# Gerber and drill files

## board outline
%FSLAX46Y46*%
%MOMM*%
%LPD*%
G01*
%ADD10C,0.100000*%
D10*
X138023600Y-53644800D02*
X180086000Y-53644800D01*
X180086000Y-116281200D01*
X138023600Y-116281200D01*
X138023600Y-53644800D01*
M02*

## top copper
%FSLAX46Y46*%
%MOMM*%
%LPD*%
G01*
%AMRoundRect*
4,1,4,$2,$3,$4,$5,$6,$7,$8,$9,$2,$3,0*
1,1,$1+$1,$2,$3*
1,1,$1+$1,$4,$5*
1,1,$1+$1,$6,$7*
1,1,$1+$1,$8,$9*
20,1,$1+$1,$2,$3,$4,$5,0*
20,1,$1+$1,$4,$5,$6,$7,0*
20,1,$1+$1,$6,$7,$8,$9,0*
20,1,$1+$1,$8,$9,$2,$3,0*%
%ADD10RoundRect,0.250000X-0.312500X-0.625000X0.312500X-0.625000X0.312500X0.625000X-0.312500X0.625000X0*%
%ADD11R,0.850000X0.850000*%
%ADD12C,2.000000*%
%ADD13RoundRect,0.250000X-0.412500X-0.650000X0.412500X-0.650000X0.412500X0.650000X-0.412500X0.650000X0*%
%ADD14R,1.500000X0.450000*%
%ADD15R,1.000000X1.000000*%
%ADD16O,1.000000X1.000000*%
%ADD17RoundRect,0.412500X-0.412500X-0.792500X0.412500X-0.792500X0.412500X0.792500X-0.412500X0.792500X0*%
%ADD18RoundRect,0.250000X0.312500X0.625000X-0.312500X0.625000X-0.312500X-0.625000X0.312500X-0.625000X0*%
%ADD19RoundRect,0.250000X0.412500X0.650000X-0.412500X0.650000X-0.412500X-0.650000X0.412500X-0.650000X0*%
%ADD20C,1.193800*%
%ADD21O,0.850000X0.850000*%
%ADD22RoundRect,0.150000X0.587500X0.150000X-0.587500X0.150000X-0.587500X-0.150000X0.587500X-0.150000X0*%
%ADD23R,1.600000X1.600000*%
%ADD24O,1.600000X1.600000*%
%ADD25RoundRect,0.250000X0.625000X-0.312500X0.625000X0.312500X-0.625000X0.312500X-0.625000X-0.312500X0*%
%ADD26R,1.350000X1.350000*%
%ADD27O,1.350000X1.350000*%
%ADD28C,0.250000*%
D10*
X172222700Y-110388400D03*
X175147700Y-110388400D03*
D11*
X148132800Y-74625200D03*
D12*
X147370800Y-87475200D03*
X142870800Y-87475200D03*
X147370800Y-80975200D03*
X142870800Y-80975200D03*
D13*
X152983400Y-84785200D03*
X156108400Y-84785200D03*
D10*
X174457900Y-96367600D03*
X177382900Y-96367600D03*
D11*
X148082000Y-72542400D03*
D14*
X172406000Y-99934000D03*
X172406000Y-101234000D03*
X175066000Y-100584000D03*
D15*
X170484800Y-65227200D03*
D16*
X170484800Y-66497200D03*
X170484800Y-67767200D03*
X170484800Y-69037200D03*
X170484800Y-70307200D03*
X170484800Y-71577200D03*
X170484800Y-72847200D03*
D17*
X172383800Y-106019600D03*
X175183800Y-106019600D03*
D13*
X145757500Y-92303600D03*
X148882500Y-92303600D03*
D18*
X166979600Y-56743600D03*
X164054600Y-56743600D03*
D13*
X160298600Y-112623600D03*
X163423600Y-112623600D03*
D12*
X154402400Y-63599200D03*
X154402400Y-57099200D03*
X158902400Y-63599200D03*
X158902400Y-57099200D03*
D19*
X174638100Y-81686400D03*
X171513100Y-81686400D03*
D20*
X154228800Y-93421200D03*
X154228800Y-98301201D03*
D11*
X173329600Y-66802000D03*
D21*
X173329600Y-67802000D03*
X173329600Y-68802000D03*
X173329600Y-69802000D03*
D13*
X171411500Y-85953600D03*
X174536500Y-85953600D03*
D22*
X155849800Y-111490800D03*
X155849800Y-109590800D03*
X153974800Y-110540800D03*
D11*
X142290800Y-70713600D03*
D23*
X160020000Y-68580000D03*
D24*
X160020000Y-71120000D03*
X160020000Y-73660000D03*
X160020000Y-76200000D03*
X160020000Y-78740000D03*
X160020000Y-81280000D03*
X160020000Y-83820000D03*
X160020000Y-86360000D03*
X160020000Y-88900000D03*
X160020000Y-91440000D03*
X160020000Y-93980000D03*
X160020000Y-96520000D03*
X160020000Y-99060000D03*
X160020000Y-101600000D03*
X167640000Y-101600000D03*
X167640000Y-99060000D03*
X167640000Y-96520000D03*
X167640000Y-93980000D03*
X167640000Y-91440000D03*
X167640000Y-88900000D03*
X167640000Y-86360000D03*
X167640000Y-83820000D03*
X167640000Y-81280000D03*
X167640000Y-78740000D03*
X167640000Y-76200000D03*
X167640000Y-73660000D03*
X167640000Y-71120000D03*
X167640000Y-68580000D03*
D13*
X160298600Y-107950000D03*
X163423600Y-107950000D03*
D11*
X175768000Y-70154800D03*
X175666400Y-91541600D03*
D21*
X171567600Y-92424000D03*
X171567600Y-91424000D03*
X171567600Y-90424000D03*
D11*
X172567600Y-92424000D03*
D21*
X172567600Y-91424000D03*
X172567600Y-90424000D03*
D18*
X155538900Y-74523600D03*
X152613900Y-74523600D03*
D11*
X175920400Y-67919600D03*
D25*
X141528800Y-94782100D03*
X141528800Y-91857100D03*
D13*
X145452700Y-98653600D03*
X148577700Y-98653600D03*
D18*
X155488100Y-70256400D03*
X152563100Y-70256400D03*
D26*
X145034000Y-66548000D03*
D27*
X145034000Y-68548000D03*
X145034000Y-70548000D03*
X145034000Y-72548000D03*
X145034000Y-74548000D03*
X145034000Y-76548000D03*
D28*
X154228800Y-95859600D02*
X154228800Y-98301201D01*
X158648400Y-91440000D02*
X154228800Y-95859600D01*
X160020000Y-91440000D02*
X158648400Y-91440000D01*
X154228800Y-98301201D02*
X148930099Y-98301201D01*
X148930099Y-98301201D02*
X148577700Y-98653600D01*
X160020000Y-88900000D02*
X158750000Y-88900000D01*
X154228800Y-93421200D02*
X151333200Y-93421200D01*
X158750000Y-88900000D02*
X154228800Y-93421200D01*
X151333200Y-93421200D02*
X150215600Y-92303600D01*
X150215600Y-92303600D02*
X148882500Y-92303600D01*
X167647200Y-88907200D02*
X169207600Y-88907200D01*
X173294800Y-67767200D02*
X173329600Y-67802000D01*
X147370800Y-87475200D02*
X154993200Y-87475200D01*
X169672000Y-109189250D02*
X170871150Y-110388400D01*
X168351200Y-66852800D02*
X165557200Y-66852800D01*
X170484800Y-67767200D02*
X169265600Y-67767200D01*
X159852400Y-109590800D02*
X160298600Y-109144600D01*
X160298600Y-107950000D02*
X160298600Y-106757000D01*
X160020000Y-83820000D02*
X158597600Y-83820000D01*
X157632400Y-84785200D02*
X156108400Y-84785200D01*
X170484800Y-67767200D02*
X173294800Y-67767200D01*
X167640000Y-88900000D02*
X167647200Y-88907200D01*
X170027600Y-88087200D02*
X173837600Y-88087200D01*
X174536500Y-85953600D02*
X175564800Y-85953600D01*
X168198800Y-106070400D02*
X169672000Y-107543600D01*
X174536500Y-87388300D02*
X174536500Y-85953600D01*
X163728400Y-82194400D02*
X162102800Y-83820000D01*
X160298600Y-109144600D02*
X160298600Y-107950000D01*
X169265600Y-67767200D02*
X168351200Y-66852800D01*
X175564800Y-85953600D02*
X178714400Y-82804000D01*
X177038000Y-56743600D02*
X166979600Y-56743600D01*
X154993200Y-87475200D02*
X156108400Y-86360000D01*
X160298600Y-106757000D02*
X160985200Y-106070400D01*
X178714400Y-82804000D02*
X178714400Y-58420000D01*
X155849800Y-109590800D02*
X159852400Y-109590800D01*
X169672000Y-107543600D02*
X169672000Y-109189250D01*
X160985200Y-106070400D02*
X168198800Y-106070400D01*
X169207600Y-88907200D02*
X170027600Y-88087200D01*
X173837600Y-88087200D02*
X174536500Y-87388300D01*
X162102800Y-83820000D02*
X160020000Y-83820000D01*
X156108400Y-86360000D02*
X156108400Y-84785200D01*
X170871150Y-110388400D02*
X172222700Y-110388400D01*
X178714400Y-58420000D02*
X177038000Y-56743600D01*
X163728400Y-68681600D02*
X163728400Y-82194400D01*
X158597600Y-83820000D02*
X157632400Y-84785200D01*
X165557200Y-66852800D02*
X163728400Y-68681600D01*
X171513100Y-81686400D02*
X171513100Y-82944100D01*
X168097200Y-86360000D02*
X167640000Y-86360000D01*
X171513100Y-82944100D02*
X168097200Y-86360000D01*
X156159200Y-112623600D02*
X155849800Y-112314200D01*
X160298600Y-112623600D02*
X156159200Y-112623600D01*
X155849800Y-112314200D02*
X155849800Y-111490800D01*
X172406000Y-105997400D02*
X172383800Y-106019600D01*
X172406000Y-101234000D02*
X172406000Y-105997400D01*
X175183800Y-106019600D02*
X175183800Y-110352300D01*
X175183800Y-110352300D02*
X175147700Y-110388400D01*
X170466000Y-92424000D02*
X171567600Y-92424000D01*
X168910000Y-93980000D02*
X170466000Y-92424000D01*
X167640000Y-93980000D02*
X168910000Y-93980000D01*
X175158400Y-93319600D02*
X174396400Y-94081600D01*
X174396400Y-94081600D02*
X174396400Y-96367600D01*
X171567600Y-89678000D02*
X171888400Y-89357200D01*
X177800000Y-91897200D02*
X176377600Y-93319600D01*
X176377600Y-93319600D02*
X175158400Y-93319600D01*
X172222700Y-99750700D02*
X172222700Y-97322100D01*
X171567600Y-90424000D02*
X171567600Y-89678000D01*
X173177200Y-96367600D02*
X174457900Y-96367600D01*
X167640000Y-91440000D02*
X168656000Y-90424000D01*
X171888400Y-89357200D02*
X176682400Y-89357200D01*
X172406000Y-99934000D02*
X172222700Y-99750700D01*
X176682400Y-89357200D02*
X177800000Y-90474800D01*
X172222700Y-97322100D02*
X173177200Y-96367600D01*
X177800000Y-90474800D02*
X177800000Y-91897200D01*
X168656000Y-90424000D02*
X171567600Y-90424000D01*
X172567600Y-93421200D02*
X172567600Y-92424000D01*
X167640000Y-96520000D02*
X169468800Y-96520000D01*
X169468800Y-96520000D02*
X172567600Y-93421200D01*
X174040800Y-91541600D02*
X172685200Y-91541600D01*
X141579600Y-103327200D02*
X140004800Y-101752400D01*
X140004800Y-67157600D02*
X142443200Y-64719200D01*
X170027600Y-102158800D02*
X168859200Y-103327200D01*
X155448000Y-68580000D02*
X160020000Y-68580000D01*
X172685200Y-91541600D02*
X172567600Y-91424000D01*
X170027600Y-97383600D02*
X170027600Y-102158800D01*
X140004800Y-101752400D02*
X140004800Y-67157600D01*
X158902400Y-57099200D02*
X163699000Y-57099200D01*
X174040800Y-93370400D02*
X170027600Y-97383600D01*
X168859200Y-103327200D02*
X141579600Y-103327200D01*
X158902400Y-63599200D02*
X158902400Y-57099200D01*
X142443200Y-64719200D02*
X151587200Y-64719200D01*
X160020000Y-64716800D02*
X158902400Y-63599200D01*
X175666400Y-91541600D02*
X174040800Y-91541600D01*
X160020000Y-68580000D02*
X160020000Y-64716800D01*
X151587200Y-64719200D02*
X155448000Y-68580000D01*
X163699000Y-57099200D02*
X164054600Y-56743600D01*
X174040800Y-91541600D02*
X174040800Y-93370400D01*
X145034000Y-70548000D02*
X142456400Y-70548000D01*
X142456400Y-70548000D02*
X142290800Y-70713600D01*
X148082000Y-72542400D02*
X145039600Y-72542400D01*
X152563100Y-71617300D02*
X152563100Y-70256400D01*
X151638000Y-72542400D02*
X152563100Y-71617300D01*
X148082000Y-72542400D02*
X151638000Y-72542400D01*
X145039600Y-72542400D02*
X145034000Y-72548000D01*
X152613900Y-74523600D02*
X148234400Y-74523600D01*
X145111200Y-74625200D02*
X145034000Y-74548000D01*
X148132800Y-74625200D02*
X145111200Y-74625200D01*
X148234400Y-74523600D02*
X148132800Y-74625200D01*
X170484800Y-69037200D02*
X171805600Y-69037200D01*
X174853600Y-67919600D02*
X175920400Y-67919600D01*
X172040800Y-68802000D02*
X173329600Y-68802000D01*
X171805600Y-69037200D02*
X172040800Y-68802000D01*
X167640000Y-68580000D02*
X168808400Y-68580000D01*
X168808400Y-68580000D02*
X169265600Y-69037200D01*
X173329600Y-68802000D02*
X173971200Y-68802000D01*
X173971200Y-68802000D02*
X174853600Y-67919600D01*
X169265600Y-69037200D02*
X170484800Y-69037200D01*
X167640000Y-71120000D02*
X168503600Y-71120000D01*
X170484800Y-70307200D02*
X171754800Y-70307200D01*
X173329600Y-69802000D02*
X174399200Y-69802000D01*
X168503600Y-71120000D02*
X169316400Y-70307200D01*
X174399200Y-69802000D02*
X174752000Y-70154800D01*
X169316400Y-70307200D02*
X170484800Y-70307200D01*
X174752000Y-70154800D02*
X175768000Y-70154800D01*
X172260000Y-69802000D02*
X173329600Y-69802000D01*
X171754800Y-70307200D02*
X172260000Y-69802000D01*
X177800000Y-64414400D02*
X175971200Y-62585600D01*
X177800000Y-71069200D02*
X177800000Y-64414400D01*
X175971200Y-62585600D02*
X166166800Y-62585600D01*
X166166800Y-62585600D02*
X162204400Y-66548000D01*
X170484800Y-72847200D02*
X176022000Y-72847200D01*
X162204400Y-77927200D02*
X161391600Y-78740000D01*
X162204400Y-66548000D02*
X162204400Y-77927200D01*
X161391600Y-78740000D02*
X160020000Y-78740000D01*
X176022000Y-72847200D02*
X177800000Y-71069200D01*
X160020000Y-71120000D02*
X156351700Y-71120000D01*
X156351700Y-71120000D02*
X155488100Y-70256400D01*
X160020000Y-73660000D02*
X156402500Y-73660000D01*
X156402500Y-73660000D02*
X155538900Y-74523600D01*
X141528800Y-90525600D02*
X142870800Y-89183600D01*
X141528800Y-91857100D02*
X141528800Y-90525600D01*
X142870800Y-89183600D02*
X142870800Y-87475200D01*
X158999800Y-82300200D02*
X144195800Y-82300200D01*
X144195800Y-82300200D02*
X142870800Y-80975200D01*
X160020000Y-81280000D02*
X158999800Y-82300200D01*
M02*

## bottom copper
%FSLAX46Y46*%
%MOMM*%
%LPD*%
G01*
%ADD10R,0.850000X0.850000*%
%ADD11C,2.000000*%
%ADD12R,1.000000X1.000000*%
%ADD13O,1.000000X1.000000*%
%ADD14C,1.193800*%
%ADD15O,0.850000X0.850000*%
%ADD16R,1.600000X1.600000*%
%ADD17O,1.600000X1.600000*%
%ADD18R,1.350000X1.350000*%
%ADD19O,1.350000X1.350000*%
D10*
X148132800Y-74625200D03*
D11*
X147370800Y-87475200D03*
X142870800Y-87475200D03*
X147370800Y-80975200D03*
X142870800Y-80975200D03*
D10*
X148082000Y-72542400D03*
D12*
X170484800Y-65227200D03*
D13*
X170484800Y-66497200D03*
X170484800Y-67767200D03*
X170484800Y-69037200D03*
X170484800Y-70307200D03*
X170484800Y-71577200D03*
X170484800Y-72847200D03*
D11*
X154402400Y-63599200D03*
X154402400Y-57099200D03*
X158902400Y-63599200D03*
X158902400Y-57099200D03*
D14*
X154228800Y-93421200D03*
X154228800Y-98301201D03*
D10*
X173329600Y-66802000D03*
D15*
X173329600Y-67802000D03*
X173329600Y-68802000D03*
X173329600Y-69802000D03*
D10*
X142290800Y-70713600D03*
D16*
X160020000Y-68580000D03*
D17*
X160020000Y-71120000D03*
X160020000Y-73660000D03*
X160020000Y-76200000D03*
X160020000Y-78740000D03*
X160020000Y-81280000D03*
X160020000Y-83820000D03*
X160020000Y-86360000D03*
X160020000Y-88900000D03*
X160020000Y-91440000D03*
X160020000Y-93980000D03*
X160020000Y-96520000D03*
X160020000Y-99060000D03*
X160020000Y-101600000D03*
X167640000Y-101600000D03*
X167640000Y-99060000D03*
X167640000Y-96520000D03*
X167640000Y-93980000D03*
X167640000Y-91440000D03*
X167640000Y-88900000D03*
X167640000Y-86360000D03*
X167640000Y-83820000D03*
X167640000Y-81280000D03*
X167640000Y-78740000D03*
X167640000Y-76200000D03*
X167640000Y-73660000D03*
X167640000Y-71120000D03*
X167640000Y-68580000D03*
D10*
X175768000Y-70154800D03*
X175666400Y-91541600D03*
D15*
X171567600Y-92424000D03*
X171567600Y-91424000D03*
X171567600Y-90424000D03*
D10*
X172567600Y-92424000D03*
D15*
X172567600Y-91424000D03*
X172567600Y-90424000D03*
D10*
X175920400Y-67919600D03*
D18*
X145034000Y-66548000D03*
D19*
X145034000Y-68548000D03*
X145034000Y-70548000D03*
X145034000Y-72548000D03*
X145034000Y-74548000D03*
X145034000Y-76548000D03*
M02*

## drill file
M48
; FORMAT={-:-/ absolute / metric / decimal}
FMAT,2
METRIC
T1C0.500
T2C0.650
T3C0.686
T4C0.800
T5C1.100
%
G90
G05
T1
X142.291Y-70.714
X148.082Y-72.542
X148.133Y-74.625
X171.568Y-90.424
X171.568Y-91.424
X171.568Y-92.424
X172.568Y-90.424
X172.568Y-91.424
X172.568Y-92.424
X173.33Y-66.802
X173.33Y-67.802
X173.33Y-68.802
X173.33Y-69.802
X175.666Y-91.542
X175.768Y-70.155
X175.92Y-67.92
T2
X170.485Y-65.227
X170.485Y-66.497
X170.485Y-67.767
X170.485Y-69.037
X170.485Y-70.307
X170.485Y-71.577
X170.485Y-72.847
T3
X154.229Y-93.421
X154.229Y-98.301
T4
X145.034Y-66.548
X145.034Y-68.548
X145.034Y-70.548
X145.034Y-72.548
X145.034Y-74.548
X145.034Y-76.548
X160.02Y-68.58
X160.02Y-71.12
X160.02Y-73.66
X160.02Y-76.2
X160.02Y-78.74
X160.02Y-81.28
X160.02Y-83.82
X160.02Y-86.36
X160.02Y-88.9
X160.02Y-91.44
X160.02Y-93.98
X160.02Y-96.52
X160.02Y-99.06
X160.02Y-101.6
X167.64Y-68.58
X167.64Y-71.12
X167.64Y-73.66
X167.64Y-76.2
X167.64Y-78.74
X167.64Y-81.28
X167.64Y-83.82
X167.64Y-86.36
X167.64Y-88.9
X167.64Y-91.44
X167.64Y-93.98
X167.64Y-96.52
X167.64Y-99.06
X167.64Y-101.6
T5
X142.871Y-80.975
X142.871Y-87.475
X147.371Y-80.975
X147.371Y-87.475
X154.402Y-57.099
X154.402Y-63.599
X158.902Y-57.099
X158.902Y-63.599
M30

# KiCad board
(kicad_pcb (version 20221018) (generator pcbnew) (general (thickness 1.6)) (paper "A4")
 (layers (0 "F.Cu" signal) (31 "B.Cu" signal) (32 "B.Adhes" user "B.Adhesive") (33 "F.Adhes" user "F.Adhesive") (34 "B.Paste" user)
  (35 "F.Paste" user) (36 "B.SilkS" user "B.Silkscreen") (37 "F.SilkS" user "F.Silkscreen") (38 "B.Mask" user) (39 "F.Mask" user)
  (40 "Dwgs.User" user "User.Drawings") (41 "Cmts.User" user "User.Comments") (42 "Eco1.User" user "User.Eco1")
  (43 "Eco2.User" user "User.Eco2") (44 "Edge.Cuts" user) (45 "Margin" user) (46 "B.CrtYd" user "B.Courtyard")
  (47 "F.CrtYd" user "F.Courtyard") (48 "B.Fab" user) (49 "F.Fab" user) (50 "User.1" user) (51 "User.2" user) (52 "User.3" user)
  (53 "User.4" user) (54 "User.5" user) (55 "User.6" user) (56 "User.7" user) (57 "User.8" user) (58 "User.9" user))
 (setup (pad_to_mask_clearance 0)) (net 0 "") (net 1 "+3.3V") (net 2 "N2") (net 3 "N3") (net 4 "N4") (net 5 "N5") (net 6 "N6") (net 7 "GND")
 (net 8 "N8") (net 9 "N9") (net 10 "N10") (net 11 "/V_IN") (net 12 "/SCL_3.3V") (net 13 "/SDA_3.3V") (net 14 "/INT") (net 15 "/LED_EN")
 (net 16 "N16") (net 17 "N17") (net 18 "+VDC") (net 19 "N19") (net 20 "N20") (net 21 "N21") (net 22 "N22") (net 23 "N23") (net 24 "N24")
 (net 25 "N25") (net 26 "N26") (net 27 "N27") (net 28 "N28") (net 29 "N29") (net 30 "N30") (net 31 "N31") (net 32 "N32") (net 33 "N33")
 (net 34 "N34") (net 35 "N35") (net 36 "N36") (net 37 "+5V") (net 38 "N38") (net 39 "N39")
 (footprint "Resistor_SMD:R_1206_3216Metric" (layer "F.Cu") (at 173.6852 110.3884)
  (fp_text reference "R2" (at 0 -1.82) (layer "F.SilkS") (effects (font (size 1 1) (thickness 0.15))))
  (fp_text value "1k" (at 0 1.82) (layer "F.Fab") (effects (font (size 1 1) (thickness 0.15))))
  (pad "1" smd roundrect (at -1.4625 0) (size 1.125 1.75) (layers "F.Cu" "F.Paste" "F.Mask") (roundrect_rratio 0.222222) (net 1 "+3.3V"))
  (pad "2" smd roundrect (at 1.4625 0) (size 1.125 1.75) (layers "F.Cu" "F.Paste" "F.Mask") (roundrect_rratio 0.222222) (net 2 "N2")))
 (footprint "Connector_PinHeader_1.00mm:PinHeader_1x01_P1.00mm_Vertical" (layer "F.Cu") (at 148.1328 74.6252)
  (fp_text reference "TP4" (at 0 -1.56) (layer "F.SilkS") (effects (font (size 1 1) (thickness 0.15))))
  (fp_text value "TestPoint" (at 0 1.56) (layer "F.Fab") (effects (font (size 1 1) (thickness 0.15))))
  (pad "1" thru_hole rect (at 0 0) (size 0.85 0.85) (drill 0.5) (layers "*.Cu" "*.Mask") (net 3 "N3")))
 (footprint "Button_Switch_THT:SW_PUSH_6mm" (layer "F.Cu") (at 147.3708 80.9752 -90)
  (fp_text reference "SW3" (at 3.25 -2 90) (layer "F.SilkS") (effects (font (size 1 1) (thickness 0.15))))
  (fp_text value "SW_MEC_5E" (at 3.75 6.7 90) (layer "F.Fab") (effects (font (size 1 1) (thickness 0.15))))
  (pad "1" thru_hole circle (at 6.5 0) (size 2 2) (drill 1.1) (layers "*.Cu" "*.Mask") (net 1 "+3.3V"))
  (pad "2" thru_hole circle (at 6.5 4.5) (size 2 2) (drill 1.1) (layers "*.Cu" "*.Mask") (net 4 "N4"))
  (pad "3" thru_hole circle (at 0 0) (size 2 2) (drill 1.1) (layers "*.Cu" "*.Mask") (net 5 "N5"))
  (pad "4" thru_hole circle (at 0 4.5) (size 2 2) (drill 1.1) (layers "*.Cu" "*.Mask") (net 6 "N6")))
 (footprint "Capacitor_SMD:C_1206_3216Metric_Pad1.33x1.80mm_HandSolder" (layer "F.Cu") (at 154.5459 84.7852)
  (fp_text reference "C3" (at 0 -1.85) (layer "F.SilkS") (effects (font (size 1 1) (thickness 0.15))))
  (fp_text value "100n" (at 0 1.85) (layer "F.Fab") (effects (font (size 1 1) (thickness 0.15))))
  (pad "1" smd roundrect (at -1.5625 0) (size 1.325 1.8) (layers "F.Cu" "F.Paste" "F.Mask") (roundrect_rratio 0.188679) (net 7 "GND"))
  (pad "2" smd roundrect (at 1.5625 0) (size 1.325 1.8) (layers "F.Cu" "F.Paste" "F.Mask") (roundrect_rratio 0.188679) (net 1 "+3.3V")))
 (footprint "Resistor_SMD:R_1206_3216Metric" (layer "F.Cu") (at 175.9204 96.3676)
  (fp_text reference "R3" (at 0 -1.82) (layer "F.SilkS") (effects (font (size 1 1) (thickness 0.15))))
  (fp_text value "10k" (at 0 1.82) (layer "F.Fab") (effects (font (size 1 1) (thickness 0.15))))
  (pad "1" smd roundrect (at -1.4625 0) (size 1.125 1.75) (layers "F.Cu" "F.Paste" "F.Mask") (roundrect_rratio 0.222222) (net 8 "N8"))
  (pad "2" smd roundrect (at 1.4625 0) (size 1.125 1.75) (layers "F.Cu" "F.Paste" "F.Mask") (roundrect_rratio 0.222222) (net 7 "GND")))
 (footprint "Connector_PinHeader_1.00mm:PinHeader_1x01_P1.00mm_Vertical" (layer "F.Cu") (at 148.082 72.5424)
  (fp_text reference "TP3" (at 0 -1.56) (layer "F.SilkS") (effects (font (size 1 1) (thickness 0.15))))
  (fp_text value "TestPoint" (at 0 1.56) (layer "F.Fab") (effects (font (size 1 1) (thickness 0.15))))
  (pad "1" thru_hole rect (at 0 0) (size 0.85 0.85) (drill 0.5) (layers "*.Cu" "*.Mask") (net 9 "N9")))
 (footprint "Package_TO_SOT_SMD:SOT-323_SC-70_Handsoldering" (layer "F.Cu") (at 173.736 100.584)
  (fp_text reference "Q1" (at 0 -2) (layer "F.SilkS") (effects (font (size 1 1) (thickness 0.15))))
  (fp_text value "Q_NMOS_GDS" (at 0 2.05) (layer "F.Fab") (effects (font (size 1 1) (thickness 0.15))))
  (pad "1" smd rect (at -1.33 -0.65 270) (size 0.45 1.5) (layers "F.Cu" "F.Paste" "F.Mask") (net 8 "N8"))
  (pad "2" smd rect (at -1.33 0.65 270) (size 0.45 1.5) (layers "F.Cu" "F.Paste" "F.Mask") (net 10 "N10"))
  (pad "3" smd rect (at 1.33 0 270) (size 0.45 1.5) (layers "F.Cu" "F.Paste" "F.Mask") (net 7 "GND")))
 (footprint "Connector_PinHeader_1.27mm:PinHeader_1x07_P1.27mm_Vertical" (layer "F.Cu") (at 170.4848 65.2272)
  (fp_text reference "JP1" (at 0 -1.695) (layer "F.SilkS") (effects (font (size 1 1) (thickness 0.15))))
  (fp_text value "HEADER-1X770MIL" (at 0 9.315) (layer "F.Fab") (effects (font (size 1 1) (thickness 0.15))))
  (pad "1" thru_hole rect (at 0 0) (size 1 1) (drill 0.65) (layers "*.Cu" "*.Mask") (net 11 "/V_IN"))
  (pad "2" thru_hole oval (at 0 1.27) (size 1 1) (drill 0.65) (layers "*.Cu" "*.Mask") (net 7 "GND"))
  (pad "3" thru_hole oval (at 0 2.54) (size 1 1) (drill 0.65) (layers "*.Cu" "*.Mask") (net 1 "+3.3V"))
  (pad "4" thru_hole oval (at 0 3.81) (size 1 1) (drill 0.65) (layers "*.Cu" "*.Mask") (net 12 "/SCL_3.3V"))
  (pad "5" thru_hole oval (at 0 5.08) (size 1 1) (drill 0.65) (layers "*.Cu" "*.Mask") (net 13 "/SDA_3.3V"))
  (pad "6" thru_hole oval (at 0 6.35) (size 1 1) (drill 0.65) (layers "*.Cu" "*.Mask") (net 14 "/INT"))
  (pad "7" thru_hole oval (at 0 7.62) (size 1 1) (drill 0.65) (layers "*.Cu" "*.Mask") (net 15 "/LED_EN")))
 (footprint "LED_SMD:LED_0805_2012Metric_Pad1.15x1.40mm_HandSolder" (layer "F.Cu") (at 173.7868 106.0196)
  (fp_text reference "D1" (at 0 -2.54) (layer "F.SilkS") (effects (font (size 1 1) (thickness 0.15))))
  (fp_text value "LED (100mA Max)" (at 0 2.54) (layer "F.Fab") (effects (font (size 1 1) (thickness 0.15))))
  (pad "1" smd roundrect (at -1.403 0) (size 1.65 2.41) (layers "F.Cu" "F.Paste" "F.Mask") (roundrect_rratio 0.25) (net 10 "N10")
   (thermal_bridge_angle 45))
  (pad "2" smd roundrect (at 1.397 0) (size 1.65 2.41) (layers "F.Cu" "F.Paste" "F.Mask") (roundrect_rratio 0.25) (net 2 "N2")
   (thermal_bridge_angle 45)))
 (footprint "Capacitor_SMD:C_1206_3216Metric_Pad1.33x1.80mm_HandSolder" (layer "F.Cu") (at 147.32 92.3036)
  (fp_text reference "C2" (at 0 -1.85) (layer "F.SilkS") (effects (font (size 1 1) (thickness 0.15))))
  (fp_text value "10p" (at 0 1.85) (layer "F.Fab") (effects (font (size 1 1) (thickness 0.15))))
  (pad "1" smd roundrect (at -1.5625 0) (size 1.325 1.8) (layers "F.Cu" "F.Paste" "F.Mask") (roundrect_rratio 0.188679) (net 7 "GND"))
  (pad "2" smd roundrect (at 1.5625 0) (size 1.325 1.8) (layers "F.Cu" "F.Paste" "F.Mask") (roundrect_rratio 0.188679) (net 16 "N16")))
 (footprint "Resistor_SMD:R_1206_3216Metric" (layer "F.Cu") (at 165.5171 56.7436 180)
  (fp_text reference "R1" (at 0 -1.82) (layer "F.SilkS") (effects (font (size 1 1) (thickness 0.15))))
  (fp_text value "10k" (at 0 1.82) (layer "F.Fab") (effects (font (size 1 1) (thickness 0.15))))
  (pad "1" smd roundrect (at -1.4625 0 180) (size 1.125 1.75) (layers "F.Cu" "F.Paste" "F.Mask") (roundrect_rratio 0.222222) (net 1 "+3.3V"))
  (pad "2" smd roundrect (at 1.4625 0 180) (size 1.125 1.75) (layers "F.Cu" "F.Paste" "F.Mask") (roundrect_rratio 0.222222) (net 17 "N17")))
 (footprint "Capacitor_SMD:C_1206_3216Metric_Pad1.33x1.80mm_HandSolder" (layer "F.Cu") (at 161.8611 112.6236)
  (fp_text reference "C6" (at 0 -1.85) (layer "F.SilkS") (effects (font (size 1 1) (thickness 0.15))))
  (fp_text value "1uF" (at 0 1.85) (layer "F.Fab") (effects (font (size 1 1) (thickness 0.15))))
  (pad "1" smd roundrect (at -1.5625 0) (size 1.325 1.8) (layers "F.Cu" "F.Paste" "F.Mask") (roundrect_rratio 0.188679) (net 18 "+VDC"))
  (pad "2" smd roundrect (at 1.5625 0) (size 1.325 1.8) (layers "F.Cu" "F.Paste" "F.Mask") (roundrect_rratio 0.188679) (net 7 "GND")))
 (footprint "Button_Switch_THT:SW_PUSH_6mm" (layer "F.Cu") (at 154.4024 63.5992 90)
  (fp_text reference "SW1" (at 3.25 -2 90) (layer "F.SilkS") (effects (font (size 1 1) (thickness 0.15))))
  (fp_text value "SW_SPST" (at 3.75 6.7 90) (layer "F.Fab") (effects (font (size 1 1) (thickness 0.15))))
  (pad "1" thru_hole circle (at 0 0 180) (size 2 2) (drill 1.1) (layers "*.Cu" "*.Mask") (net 7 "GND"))
  (pad "1" thru_hole circle (at 6.5 0 180) (size 2 2) (drill 1.1) (layers "*.Cu" "*.Mask") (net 7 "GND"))
  (pad "2" thru_hole circle (at 0 4.5 180) (size 2 2) (drill 1.1) (layers "*.Cu" "*.Mask") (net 17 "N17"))
  (pad "2" thru_hole circle (at 6.5 4.5 180) (size 2 2) (drill 1.1) (layers "*.Cu" "*.Mask") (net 17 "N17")))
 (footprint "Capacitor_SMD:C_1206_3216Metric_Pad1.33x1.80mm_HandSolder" (layer "F.Cu") (at 173.0756 81.6864 180)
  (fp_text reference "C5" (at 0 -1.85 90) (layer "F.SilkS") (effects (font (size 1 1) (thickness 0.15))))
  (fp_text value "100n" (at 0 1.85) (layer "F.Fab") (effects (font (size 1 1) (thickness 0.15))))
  (pad "1" smd roundrect (at -1.5625 0 180) (size 1.325 1.8) (layers "F.Cu" "F.Paste" "F.Mask") (roundrect_rratio 0.188679) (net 7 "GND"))
  (pad "2" smd roundrect (at 1.5625 0 180) (size 1.325 1.8) (layers "F.Cu" "F.Paste" "F.Mask") (roundrect_rratio 0.188679) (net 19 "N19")))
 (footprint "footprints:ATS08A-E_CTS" (layer "F.Cu") (at 154.2288 93.4212 -90)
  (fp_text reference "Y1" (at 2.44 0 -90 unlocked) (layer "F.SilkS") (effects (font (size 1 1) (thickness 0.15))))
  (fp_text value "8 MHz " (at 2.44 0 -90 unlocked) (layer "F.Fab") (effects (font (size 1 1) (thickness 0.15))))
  (pad "1" thru_hole circle (at 0 0 270) (size 1.1938 1.1938) (drill 0.6858) (layers "*.Cu" "*.Mask") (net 16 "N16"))
  (pad "2" thru_hole circle (at 4.880001 0 270) (size 1.1938 1.1938) (drill 0.6858) (layers "*.Cu" "*.Mask") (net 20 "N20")))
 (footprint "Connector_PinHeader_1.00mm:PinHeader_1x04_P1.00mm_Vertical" (layer "F.Cu") (at 173.3296 66.802)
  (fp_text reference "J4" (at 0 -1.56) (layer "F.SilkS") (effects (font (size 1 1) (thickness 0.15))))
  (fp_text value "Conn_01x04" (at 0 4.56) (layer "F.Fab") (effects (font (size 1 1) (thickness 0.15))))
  (pad "1" thru_hole rect (at 0 0) (size 0.85 0.85) (drill 0.5) (layers "*.Cu" "*.Mask") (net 7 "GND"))
  (pad "2" thru_hole oval (at 0 1) (size 0.85 0.85) (drill 0.5) (layers "*.Cu" "*.Mask") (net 1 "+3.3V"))
  (pad "3" thru_hole oval (at 0 2) (size 0.85 0.85) (drill 0.5) (layers "*.Cu" "*.Mask") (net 12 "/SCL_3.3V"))
  (pad "4" thru_hole oval (at 0 3) (size 0.85 0.85) (drill 0.5) (layers "*.Cu" "*.Mask") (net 13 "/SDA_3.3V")))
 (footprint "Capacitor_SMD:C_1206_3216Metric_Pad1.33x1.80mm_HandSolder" (layer "F.Cu") (at 172.974 85.9536)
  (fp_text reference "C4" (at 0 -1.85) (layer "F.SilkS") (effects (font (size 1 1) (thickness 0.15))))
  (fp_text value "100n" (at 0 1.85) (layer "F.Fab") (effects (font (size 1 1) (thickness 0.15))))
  (pad "1" smd roundrect (at -1.5625 0) (size 1.325 1.8) (layers "F.Cu" "F.Paste" "F.Mask") (roundrect_rratio 0.188679) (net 7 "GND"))
  (pad "2" smd roundrect (at 1.5625 0) (size 1.325 1.8) (layers "F.Cu" "F.Paste" "F.Mask") (roundrect_rratio 0.188679) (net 1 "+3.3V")))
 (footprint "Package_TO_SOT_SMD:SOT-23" (layer "F.Cu") (at 154.9123 110.5408 180)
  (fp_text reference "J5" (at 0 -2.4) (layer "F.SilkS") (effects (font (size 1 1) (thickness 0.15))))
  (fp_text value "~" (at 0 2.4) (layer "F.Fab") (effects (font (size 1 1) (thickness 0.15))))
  (pad "1" smd roundrect (at -0.9375 -0.95 180) (size 1.475 0.6) (layers "F.Cu" "F.Paste" "F.Mask") (roundrect_rratio 0.25) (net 18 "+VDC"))
  (pad "2" smd roundrect (at -0.9375 0.95 180) (size 1.475 0.6) (layers "F.Cu" "F.Paste" "F.Mask") (roundrect_rratio 0.25) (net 1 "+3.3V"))
  (pad "3" smd roundrect (at 0.9375 0 180) (size 1.475 0.6) (layers "F.Cu" "F.Paste" "F.Mask") (roundrect_rratio 0.25) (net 7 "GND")))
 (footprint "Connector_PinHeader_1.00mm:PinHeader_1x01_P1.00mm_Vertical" (layer "F.Cu") (at 142.2908 70.7136)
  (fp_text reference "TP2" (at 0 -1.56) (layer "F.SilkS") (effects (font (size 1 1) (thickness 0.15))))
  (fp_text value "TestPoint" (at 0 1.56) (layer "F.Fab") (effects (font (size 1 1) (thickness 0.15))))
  (pad "1" thru_hole rect (at 0 0) (size 0.85 0.85) (drill 0.5) (layers "*.Cu" "*.Mask") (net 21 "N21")))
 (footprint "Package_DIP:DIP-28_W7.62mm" (layer "F.Cu") (at 160.02 68.58)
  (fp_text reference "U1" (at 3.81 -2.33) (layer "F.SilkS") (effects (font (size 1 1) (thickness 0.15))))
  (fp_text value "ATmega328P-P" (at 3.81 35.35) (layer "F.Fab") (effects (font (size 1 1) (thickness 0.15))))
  (pad "1" thru_hole rect (at 0 0) (size 1.6 1.6) (drill 0.8) (layers "*.Cu" "*.Mask") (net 17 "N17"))
  (pad "2" thru_hole oval (at 0 2.54) (size 1.6 1.6) (drill 0.8) (layers "*.Cu" "*.Mask") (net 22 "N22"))
  (pad "3" thru_hole oval (at 0 5.08) (size 1.6 1.6) (drill 0.8) (layers "*.Cu" "*.Mask") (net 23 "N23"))
  (pad "4" thru_hole oval (at 0 7.62) (size 1.6 1.6) (drill 0.8) (layers "*.Cu" "*.Mask") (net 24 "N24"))
  (pad "5" thru_hole oval (at 0 10.16) (size 1.6 1.6) (drill 0.8) (layers "*.Cu" "*.Mask") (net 15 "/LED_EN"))
  (pad "6" thru_hole oval (at 0 12.7) (size 1.6 1.6) (drill 0.8) (layers "*.Cu" "*.Mask") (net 6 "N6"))
  (pad "7" thru_hole oval (at 0 15.24) (size 1.6 1.6) (drill 0.8) (layers "*.Cu" "*.Mask") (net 1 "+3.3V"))
  (pad "8" thru_hole oval (at 0 17.78) (size 1.6 1.6) (drill 0.8) (layers "*.Cu" "*.Mask") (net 7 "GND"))
  (pad "9" thru_hole oval (at 0 20.32) (size 1.6 1.6) (drill 0.8) (layers "*.Cu" "*.Mask") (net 16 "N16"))
  (pad "10" thru_hole oval (at 0 22.86) (size 1.6 1.6) (drill 0.8) (layers "*.Cu" "*.Mask") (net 20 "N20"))
  (pad "11" thru_hole oval (at 0 25.4) (size 1.6 1.6) (drill 0.8) (layers "*.Cu" "*.Mask") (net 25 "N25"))
  (pad "12" thru_hole oval (at 0 27.94) (size 1.6 1.6) (drill 0.8) (layers "*.Cu" "*.Mask") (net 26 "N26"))
  (pad "13" thru_hole oval (at 0 30.48) (size 1.6 1.6) (drill 0.8) (layers "*.Cu" "*.Mask") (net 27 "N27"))
  (pad "14" thru_hole oval (at 0 33.02) (size 1.6 1.6) (drill 0.8) (layers "*.Cu" "*.Mask") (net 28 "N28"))
  (pad "15" thru_hole oval (at 7.62 33.02) (size 1.6 1.6) (drill 0.8) (layers "*.Cu" "*.Mask") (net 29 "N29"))
  (pad "16" thru_hole oval (at 7.62 30.48) (size 1.6 1.6) (drill 0.8) (layers "*.Cu" "*.Mask") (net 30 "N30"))
  (pad "17" thru_hole oval (at 7.62 27.94) (size 1.6 1.6) (drill 0.8) (layers "*.Cu" "*.Mask") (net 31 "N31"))
  (pad "18" thru_hole oval (at 7.62 25.4) (size 1.6 1.6) (drill 0.8) (layers "*.Cu" "*.Mask") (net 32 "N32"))
  (pad "19" thru_hole oval (at 7.62 22.86) (size 1.6 1.6) (drill 0.8) (layers "*.Cu" "*.Mask") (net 8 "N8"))
  (pad "20" thru_hole oval (at 7.62 20.32) (size 1.6 1.6) (drill 0.8) (layers "*.Cu" "*.Mask") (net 1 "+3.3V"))
  (pad "21" thru_hole oval (at 7.62 17.78) (size 1.6 1.6) (drill 0.8) (layers "*.Cu" "*.Mask") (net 19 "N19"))
  (pad "22" thru_hole oval (at 7.62 15.24) (size 1.6 1.6) (drill 0.8) (layers "*.Cu" "*.Mask") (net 7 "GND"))
  (pad "23" thru_hole oval (at 7.62 12.7) (size 1.6 1.6) (drill 0.8) (layers "*.Cu" "*.Mask") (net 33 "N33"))
  (pad "24" thru_hole oval (at 7.62 10.16) (size 1.6 1.6) (drill 0.8) (layers "*.Cu" "*.Mask") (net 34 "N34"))
  (pad "25" thru_hole oval (at 7.62 7.62) (size 1.6 1.6) (drill 0.8) (layers "*.Cu" "*.Mask") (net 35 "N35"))
  (pad "26" thru_hole oval (at 7.62 5.08) (size 1.6 1.6) (drill 0.8) (layers "*.Cu" "*.Mask") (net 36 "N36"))
  (pad "27" thru_hole oval (at 7.62 2.54) (size 1.6 1.6) (drill 0.8) (layers "*.Cu" "*.Mask") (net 13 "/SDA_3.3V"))
  (pad "28" thru_hole oval (at 7.62 0) (size 1.6 1.6) (drill 0.8) (layers "*.Cu" "*.Mask") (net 12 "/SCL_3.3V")))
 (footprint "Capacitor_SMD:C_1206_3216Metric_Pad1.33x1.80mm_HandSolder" (layer "F.Cu") (at 161.8611 107.95)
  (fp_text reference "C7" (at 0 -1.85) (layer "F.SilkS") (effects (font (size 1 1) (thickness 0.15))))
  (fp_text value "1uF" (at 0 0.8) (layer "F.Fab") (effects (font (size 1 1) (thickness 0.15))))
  (pad "1" smd roundrect (at -1.5625 0) (size 1.325 1.8) (layers "F.Cu" "F.Paste" "F.Mask") (roundrect_rratio 0.188679) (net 1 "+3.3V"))
  (pad "2" smd roundrect (at 1.5625 0) (size 1.325 1.8) (layers "F.Cu" "F.Paste" "F.Mask") (roundrect_rratio 0.188679) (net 7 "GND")))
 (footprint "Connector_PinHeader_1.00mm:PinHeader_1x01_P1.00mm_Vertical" (layer "F.Cu") (at 175.768 70.1548)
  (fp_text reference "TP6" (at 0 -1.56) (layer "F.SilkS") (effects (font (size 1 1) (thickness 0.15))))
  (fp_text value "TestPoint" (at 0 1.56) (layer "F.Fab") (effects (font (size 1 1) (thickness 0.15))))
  (pad "1" thru_hole rect (at 0 0) (size 0.85 0.85) (drill 0.5) (layers "*.Cu" "*.Mask") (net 13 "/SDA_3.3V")))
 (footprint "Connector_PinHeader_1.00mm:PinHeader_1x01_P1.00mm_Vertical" (layer "F.Cu") (at 175.6664 91.5416)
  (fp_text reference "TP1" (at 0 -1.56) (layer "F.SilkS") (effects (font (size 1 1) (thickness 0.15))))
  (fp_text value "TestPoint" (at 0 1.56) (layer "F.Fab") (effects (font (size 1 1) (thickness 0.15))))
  (pad "1" thru_hole rect (at 0 0) (size 0.85 0.85) (drill 0.5) (layers "*.Cu" "*.Mask") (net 17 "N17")))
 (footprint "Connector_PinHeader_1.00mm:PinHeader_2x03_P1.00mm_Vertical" (layer "F.Cu") (at 172.5676 92.424 180)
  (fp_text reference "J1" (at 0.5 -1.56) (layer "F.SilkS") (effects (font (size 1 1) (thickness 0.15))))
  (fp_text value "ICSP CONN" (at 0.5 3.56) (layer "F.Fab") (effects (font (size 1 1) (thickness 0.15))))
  (pad "1" thru_hole oval (at 1 0 180) (size 0.85 0.85) (drill 0.5) (layers "*.Cu" "*.Mask") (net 32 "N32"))
  (pad "2" thru_hole oval (at 1 1 180) (size 0.85 0.85) (drill 0.5) (layers "*.Cu" "*.Mask") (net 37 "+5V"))
  (pad "3" thru_hole oval (at 1 2 180) (size 0.85 0.85) (drill 0.5) (layers "*.Cu" "*.Mask") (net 8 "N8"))
  (pad "4" thru_hole rect (at 0 0 180) (size 0.85 0.85) (drill 0.5) (layers "*.Cu" "*.Mask") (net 31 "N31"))
  (pad "5" thru_hole oval (at 0 1 180) (size 0.85 0.85) (drill 0.5) (layers "*.Cu" "*.Mask") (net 17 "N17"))
  (pad "6" thru_hole oval (at 0 2 180) (size 0.85 0.85) (drill 0.5) (layers "*.Cu" "*.Mask") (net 7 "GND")))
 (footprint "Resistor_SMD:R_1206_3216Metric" (layer "F.Cu") (at 154.0764 74.5236 180)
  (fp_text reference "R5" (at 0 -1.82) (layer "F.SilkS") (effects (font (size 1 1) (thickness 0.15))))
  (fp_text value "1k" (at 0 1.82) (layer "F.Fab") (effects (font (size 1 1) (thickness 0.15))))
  (pad "1" smd roundrect (at -1.4625 0 180) (size 1.125 1.75) (layers "F.Cu" "F.Paste" "F.Mask") (roundrect_rratio 0.222222) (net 23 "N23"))
  (pad "2" smd roundrect (at 1.4625 0 180) (size 1.125 1.75) (layers "F.Cu" "F.Paste" "F.Mask") (roundrect_rratio 0.222222) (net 3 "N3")))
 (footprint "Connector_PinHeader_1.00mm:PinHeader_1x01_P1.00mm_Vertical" (layer "F.Cu") (at 175.9204 67.9196)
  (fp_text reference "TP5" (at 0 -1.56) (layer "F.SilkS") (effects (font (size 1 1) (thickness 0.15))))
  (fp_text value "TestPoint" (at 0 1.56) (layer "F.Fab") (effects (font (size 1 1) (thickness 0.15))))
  (pad "1" thru_hole rect (at 0 0) (size 0.85 0.85) (drill 0.5) (layers "*.Cu" "*.Mask") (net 12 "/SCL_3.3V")))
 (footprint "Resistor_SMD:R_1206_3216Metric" (layer "F.Cu") (at 141.5288 93.3196 90)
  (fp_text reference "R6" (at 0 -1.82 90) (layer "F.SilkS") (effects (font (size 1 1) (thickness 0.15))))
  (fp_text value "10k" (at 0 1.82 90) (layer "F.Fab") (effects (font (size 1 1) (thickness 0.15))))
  (pad "1" smd roundrect (at -1.4625 0 90) (size 1.125 1.75) (layers "F.Cu" "F.Paste" "F.Mask") (roundrect_rratio 0.222222) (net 7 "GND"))
  (pad "2" smd roundrect (at 1.4625 0 90) (size 1.125 1.75) (layers "F.Cu" "F.Paste" "F.Mask") (roundrect_rratio 0.222222) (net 4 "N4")))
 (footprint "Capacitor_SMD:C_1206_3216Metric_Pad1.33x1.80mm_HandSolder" (layer "F.Cu") (at 147.0152 98.6536)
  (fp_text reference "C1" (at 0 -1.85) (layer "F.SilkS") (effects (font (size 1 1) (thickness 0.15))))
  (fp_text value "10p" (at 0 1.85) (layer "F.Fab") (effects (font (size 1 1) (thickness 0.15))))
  (pad "1" smd roundrect (at -1.5625 0) (size 1.325 1.8) (layers "F.Cu" "F.Paste" "F.Mask") (roundrect_rratio 0.188679) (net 7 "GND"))
  (pad "2" smd roundrect (at 1.5625 0) (size 1.325 1.8) (layers "F.Cu" "F.Paste" "F.Mask") (roundrect_rratio 0.188679) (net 20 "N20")))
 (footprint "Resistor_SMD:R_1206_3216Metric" (layer "F.Cu") (at 154.0256 70.2564 180)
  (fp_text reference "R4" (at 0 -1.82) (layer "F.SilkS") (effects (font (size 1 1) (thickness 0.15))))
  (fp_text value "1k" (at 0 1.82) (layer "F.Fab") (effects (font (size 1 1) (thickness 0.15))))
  (pad "1" smd roundrect (at -1.4625 0 180) (size 1.125 1.75) (layers "F.Cu" "F.Paste" "F.Mask") (roundrect_rratio 0.222222) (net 22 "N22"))
  (pad "2" smd roundrect (at 1.4625 0 180) (size 1.125 1.75) (layers "F.Cu" "F.Paste" "F.Mask") (roundrect_rratio 0.222222) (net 9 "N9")))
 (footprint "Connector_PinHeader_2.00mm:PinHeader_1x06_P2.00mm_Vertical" (layer "F.Cu") (at 145.034 66.548)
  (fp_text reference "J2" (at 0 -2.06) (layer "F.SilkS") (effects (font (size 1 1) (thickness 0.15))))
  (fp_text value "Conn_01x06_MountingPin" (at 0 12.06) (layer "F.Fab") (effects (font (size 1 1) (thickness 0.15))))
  (pad "1" thru_hole rect (at 0 0) (size 1.35 1.35) (drill 0.8) (layers "*.Cu" "*.Mask") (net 7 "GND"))
  (pad "2" thru_hole oval (at 0 2) (size 1.35 1.35) (drill 0.8) (layers "*.Cu" "*.Mask") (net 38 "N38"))
  (pad "3" thru_hole oval (at 0 4) (size 1.35 1.35) (drill 0.8) (layers "*.Cu" "*.Mask") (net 21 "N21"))
  (pad "4" thru_hole oval (at 0 6) (size 1.35 1.35) (drill 0.8) (layers "*.Cu" "*.Mask") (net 9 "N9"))
  (pad "5" thru_hole oval (at 0 8) (size 1.35 1.35) (drill 0.8) (layers "*.Cu" "*.Mask") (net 3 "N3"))
  (pad "6" thru_hole oval (at 0 10) (size 1.35 1.35) (drill 0.8) (layers "*.Cu" "*.Mask") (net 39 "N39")))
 (gr_rect (start 138.0236 53.6448) (end 180.086 116.2812) (stroke (width 0.1) (type default)) (fill none) (layer "Edge.Cuts"))
 (segment (start 154.2288 95.8596) (end 154.2288 98.301201) (width 0.25) (layer "F.Cu") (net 20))
 (segment (start 158.6484 91.44) (end 154.2288 95.8596) (width 0.25) (layer "F.Cu") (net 20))
 (segment (start 160.02 91.44) (end 158.6484 91.44) (width 0.25) (layer "F.Cu") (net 20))
 (segment (start 154.2288 98.301201) (end 148.930099 98.301201) (width 0.25) (layer "F.Cu") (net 20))
 (segment (start 148.930099 98.301201) (end 148.5777 98.6536) (width 0.25) (layer "F.Cu") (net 20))
 (segment (start 160.02 88.9) (end 158.75 88.9) (width 0.25) (layer "F.Cu") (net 16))
 (segment (start 154.2288 93.4212) (end 151.3332 93.4212) (width 0.25) (layer "F.Cu") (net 16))
 (segment (start 158.75 88.9) (end 154.2288 93.4212) (width 0.25) (layer "F.Cu") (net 16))
 (segment (start 151.3332 93.4212) (end 150.2156 92.3036) (width 0.25) (layer "F.Cu") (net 16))
 (segment (start 150.2156 92.3036) (end 148.8825 92.3036) (width 0.25) (layer "F.Cu") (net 16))
 (segment (start 167.6472 88.9072) (end 169.2076 88.9072) (width 0.25) (layer "F.Cu") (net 1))
 (segment (start 173.2948 67.7672) (end 173.3296 67.802) (width 0.25) (layer "F.Cu") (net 1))
 (segment (start 147.3708 87.4752) (end 154.9932 87.4752) (width 0.25) (layer "F.Cu") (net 1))
 (segment (start 169.672 109.18925) (end 170.87115 110.3884) (width 0.25) (layer "F.Cu") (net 1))
 (segment (start 168.3512 66.8528) (end 165.5572 66.8528) (width 0.25) (layer "F.Cu") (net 1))
 (segment (start 170.4848 67.7672) (end 169.2656 67.7672) (width 0.25) (layer "F.Cu") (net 1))
 (segment (start 159.8524 109.5908) (end 160.2986 109.1446) (width 0.25) (layer "F.Cu") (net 1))
 (segment (start 160.2986 107.95) (end 160.2986 106.757) (width 0.25) (layer "F.Cu") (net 1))
 (segment (start 160.02 83.82) (end 158.5976 83.82) (width 0.25) (layer "F.Cu") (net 1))
 (segment (start 157.6324 84.7852) (end 156.1084 84.7852) (width 0.25) (layer "F.Cu") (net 1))
 (segment (start 170.4848 67.7672) (end 173.2948 67.7672) (width 0.25) (layer "F.Cu") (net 1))
 (segment (start 167.64 88.9) (end 167.6472 88.9072) (width 0.25) (layer "F.Cu") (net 1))
 (segment (start 170.0276 88.0872) (end 173.8376 88.0872) (width 0.25) (layer "F.Cu") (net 1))
 (segment (start 174.5365 85.9536) (end 175.5648 85.9536) (width 0.25) (layer "F.Cu") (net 1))
 (segment (start 168.1988 106.0704) (end 169.672 107.5436) (width 0.25) (layer "F.Cu") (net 1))
 (segment (start 174.5365 87.3883) (end 174.5365 85.9536) (width 0.25) (layer "F.Cu") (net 1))
 (segment (start 163.7284 82.1944) (end 162.1028 83.82) (width 0.25) (layer "F.Cu") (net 1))
 (segment (start 160.2986 109.1446) (end 160.2986 107.95) (width 0.25) (layer "F.Cu") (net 1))
 (segment (start 169.2656 67.7672) (end 168.3512 66.8528) (width 0.25) (layer "F.Cu") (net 1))
 (segment (start 175.5648 85.9536) (end 178.7144 82.804) (width 0.25) (layer "F.Cu") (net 1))
 (segment (start 177.038 56.7436) (end 166.9796 56.7436) (width 0.25) (layer "F.Cu") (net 1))
 (segment (start 154.9932 87.4752) (end 156.1084 86.36) (width 0.25) (layer "F.Cu") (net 1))
 (segment (start 160.2986 106.757) (end 160.9852 106.0704) (width 0.25) (layer "F.Cu") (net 1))
 (segment (start 178.7144 82.804) (end 178.7144 58.42) (width 0.25) (layer "F.Cu") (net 1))
 (segment (start 155.8498 109.5908) (end 159.8524 109.5908) (width 0.25) (layer "F.Cu") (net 1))
 (segment (start 169.672 107.5436) (end 169.672 109.18925) (width 0.25) (layer "F.Cu") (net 1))
 (segment (start 160.9852 106.0704) (end 168.1988 106.0704) (width 0.25) (layer "F.Cu") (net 1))
 (segment (start 169.2076 88.9072) (end 170.0276 88.0872) (width 0.25) (layer "F.Cu") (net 1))
 (segment (start 173.8376 88.0872) (end 174.5365 87.3883) (width 0.25) (layer "F.Cu") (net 1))
 (segment (start 162.1028 83.82) (end 160.02 83.82) (width 0.25) (layer "F.Cu") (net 1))
 (segment (start 156.1084 86.36) (end 156.1084 84.7852) (width 0.25) (layer "F.Cu") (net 1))
 (segment (start 170.87115 110.3884) (end 172.2227 110.3884) (width 0.25) (layer "F.Cu") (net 1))
 (segment (start 178.7144 58.42) (end 177.038 56.7436) (width 0.25) (layer "F.Cu") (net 1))
 (segment (start 163.7284 68.6816) (end 163.7284 82.1944) (width 0.25) (layer "F.Cu") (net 1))
 (segment (start 158.5976 83.82) (end 157.6324 84.7852) (width 0.25) (layer "F.Cu") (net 1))
 (segment (start 165.5572 66.8528) (end 163.7284 68.6816) (width 0.25) (layer "F.Cu") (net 1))
 (segment (start 171.5131 81.6864) (end 171.5131 82.9441) (width 0.25) (layer "F.Cu") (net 19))
 (segment (start 168.0972 86.36) (end 167.64 86.36) (width 0.25) (layer "F.Cu") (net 19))
 (segment (start 171.5131 82.9441) (end 168.0972 86.36) (width 0.25) (layer "F.Cu") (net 19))
 (segment (start 156.1592 112.6236) (end 155.8498 112.3142) (width 0.25) (layer "F.Cu") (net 18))
 (segment (start 160.2986 112.6236) (end 156.1592 112.6236) (width 0.25) (layer "F.Cu") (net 18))
 (segment (start 155.8498 112.3142) (end 155.8498 111.4908) (width 0.25) (layer "F.Cu") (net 18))
 (segment (start 172.406 105.9974) (end 172.3838 106.0196) (width 0.25) (layer "F.Cu") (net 10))
 (segment (start 172.406 101.234) (end 172.406 105.9974) (width 0.25) (layer "F.Cu") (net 10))
 (segment (start 175.1838 106.0196) (end 175.1838 110.3523) (width 0.25) (layer "F.Cu") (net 2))
 (segment (start 175.1838 110.3523) (end 175.1477 110.3884) (width 0.25) (layer "F.Cu") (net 2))
 (segment (start 170.466 92.424) (end 171.5676 92.424) (width 0.25) (layer "F.Cu") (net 32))
 (segment (start 168.91 93.98) (end 170.466 92.424) (width 0.25) (layer "F.Cu") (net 32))
 (segment (start 167.64 93.98) (end 168.91 93.98) (width 0.25) (layer "F.Cu") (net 32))
 (segment (start 175.1584 93.3196) (end 174.3964 94.0816) (width 0.25) (layer "F.Cu") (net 8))
 (segment (start 174.3964 94.0816) (end 174.3964 96.3676) (width 0.25) (layer "F.Cu") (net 8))
 (segment (start 171.5676 89.678) (end 171.8884 89.3572) (width 0.25) (layer "F.Cu") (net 8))
 (segment (start 177.8 91.8972) (end 176.3776 93.3196) (width 0.25) (layer "F.Cu") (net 8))
 (segment (start 176.3776 93.3196) (end 175.1584 93.3196) (width 0.25) (layer "F.Cu") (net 8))
 (segment (start 172.2227 99.7507) (end 172.2227 97.3221) (width 0.25) (layer "F.Cu") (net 8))
 (segment (start 171.5676 90.424) (end 171.5676 89.678) (width 0.25) (layer "F.Cu") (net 8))
 (segment (start 173.1772 96.3676) (end 174.4579 96.3676) (width 0.25) (layer "F.Cu") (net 8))
 (segment (start 167.64 91.44) (end 168.656 90.424) (width 0.25) (layer "F.Cu") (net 8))
 (segment (start 171.8884 89.3572) (end 176.6824 89.3572) (width 0.25) (layer "F.Cu") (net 8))
 (segment (start 172.406 99.934) (end 172.2227 99.7507) (width 0.25) (layer "F.Cu") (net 8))
 (segment (start 176.6824 89.3572) (end 177.8 90.4748) (width 0.25) (layer "F.Cu") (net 8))
 (segment (start 172.2227 97.3221) (end 173.1772 96.3676) (width 0.25) (layer "F.Cu") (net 8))
 (segment (start 177.8 90.4748) (end 177.8 91.8972) (width 0.25) (layer "F.Cu") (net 8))
 (segment (start 168.656 90.424) (end 171.5676 90.424) (width 0.25) (layer "F.Cu") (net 8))
 (segment (start 172.5676 93.4212) (end 172.5676 92.424) (width 0.25) (layer "F.Cu") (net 31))
 (segment (start 167.64 96.52) (end 169.4688 96.52) (width 0.25) (layer "F.Cu") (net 31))
 (segment (start 169.4688 96.52) (end 172.5676 93.4212) (width 0.25) (layer "F.Cu") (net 31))
 (segment (start 174.0408 91.5416) (end 172.6852 91.5416) (width 0.25) (layer "F.Cu") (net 17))
 (segment (start 141.5796 103.3272) (end 140.0048 101.7524) (width 0.25) (layer "F.Cu") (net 17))
 (segment (start 140.0048 67.1576) (end 142.4432 64.7192) (width 0.25) (layer "F.Cu") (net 17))
 (segment (start 170.0276 102.1588) (end 168.8592 103.3272) (width 0.25) (layer "F.Cu") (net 17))
 (segment (start 155.448 68.58) (end 160.02 68.58) (width 0.25) (layer "F.Cu") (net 17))
 (segment (start 172.6852 91.5416) (end 172.5676 91.424) (width 0.25) (layer "F.Cu") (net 17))
 (segment (start 170.0276 97.3836) (end 170.0276 102.1588) (width 0.25) (layer "F.Cu") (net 17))
 (segment (start 140.0048 101.7524) (end 140.0048 67.1576) (width 0.25) (layer "F.Cu") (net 17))
 (segment (start 158.9024 57.0992) (end 163.699 57.0992) (width 0.25) (layer "F.Cu") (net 17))
 (segment (start 174.0408 93.3704) (end 170.0276 97.3836) (width 0.25) (layer "F.Cu") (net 17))
 (segment (start 168.8592 103.3272) (end 141.5796 103.3272) (width 0.25) (layer "F.Cu") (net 17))
 (segment (start 158.9024 63.5992) (end 158.9024 57.0992) (width 0.25) (layer "F.Cu") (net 17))
 (segment (start 142.4432 64.7192) (end 151.5872 64.7192) (width 0.25) (layer "F.Cu") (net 17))
 (segment (start 160.02 64.7168) (end 158.9024 63.5992) (width 0.25) (layer "F.Cu") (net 17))
 (segment (start 175.6664 91.5416) (end 174.0408 91.5416) (width 0.25) (layer "F.Cu") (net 17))
 (segment (start 160.02 68.58) (end 160.02 64.7168) (width 0.25) (layer "F.Cu") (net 17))
 (segment (start 151.5872 64.7192) (end 155.448 68.58) (width 0.25) (layer "F.Cu") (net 17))
 (segment (start 163.699 57.0992) (end 164.0546 56.7436) (width 0.25) (layer "F.Cu") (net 17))
 (segment (start 174.0408 91.5416) (end 174.0408 93.3704) (width 0.25) (layer "F.Cu") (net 17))
 (segment (start 145.034 70.548) (end 142.4564 70.548) (width 0.25) (layer "F.Cu") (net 21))
 (segment (start 142.4564 70.548) (end 142.2908 70.7136) (width 0.25) (layer "F.Cu") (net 21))
 (segment (start 148.082 72.5424) (end 145.0396 72.5424) (width 0.25) (layer "F.Cu") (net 9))
 (segment (start 152.5631 71.6173) (end 152.5631 70.2564) (width 0.25) (layer "F.Cu") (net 9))
 (segment (start 151.638 72.5424) (end 152.5631 71.6173) (width 0.25) (layer "F.Cu") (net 9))
 (segment (start 148.082 72.5424) (end 151.638 72.5424) (width 0.25) (layer "F.Cu") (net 9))
 (segment (start 145.0396 72.5424) (end 145.034 72.548) (width 0.25) (layer "F.Cu") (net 9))
 (segment (start 152.6139 74.5236) (end 148.2344 74.5236) (width 0.25) (layer "F.Cu") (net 3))
 (segment (start 145.1112 74.6252) (end 145.034 74.548) (width 0.25) (layer "F.Cu") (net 3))
 (segment (start 148.1328 74.6252) (end 145.1112 74.6252) (width 0.25) (layer "F.Cu") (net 3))
 (segment (start 148.2344 74.5236) (end 148.1328 74.6252) (width 0.25) (layer "F.Cu") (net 3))
 (segment (start 170.4848 69.0372) (end 171.8056 69.0372) (width 0.25) (layer "F.Cu") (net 12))
 (segment (start 174.8536 67.9196) (end 175.9204 67.9196) (width 0.25) (layer "F.Cu") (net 12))
 (segment (start 172.0408 68.802) (end 173.3296 68.802) (width 0.25) (layer "F.Cu") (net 12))
 (segment (start 171.8056 69.0372) (end 172.0408 68.802) (width 0.25) (layer "F.Cu") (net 12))
 (segment (start 167.64 68.58) (end 168.8084 68.58) (width 0.25) (layer "F.Cu") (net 12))
 (segment (start 168.8084 68.58) (end 169.2656 69.0372) (width 0.25) (layer "F.Cu") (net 12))
 (segment (start 173.3296 68.802) (end 173.9712 68.802) (width 0.25) (layer "F.Cu") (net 12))
 (segment (start 173.9712 68.802) (end 174.8536 67.9196) (width 0.25) (layer "F.Cu") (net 12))
 (segment (start 169.2656 69.0372) (end 170.4848 69.0372) (width 0.25) (layer "F.Cu") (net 12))
 (segment (start 167.64 71.12) (end 168.5036 71.12) (width 0.25) (layer "F.Cu") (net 13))
 (segment (start 170.4848 70.3072) (end 171.7548 70.3072) (width 0.25) (layer "F.Cu") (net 13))
 (segment (start 173.3296 69.802) (end 174.3992 69.802) (width 0.25) (layer "F.Cu") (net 13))
 (segment (start 168.5036 71.12) (end 169.3164 70.3072) (width 0.25) (layer "F.Cu") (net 13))
 (segment (start 174.3992 69.802) (end 174.752 70.1548) (width 0.25) (layer "F.Cu") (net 13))
 (segment (start 169.3164 70.3072) (end 170.4848 70.3072) (width 0.25) (layer "F.Cu") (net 13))
 (segment (start 174.752 70.1548) (end 175.768 70.1548) (width 0.25) (layer "F.Cu") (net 13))
 (segment (start 172.26 69.802) (end 173.3296 69.802) (width 0.25) (layer "F.Cu") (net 13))
 (segment (start 171.7548 70.3072) (end 172.26 69.802) (width 0.25) (layer "F.Cu") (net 13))
 (segment (start 177.8 64.4144) (end 175.9712 62.5856) (width 0.25) (layer "F.Cu") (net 15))
 (segment (start 177.8 71.0692) (end 177.8 64.4144) (width 0.25) (layer "F.Cu") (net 15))
 (segment (start 175.9712 62.5856) (end 166.1668 62.5856) (width 0.25) (layer "F.Cu") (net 15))
 (segment (start 166.1668 62.5856) (end 162.2044 66.548) (width 0.25) (layer "F.Cu") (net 15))
 (segment (start 170.4848 72.8472) (end 176.022 72.8472) (width 0.25) (layer "F.Cu") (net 15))
 (segment (start 162.2044 77.9272) (end 161.3916 78.74) (width 0.25) (layer "F.Cu") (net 15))
 (segment (start 162.2044 66.548) (end 162.2044 77.9272) (width 0.25) (layer "F.Cu") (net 15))
 (segment (start 161.3916 78.74) (end 160.02 78.74) (width 0.25) (layer "F.Cu") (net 15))
 (segment (start 176.022 72.8472) (end 177.8 71.0692) (width 0.25) (layer "F.Cu") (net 15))
 (segment (start 160.02 71.12) (end 156.3517 71.12) (width 0.25) (layer "F.Cu") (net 22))
 (segment (start 156.3517 71.12) (end 155.4881 70.2564) (width 0.25) (layer "F.Cu") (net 22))
 (segment (start 160.02 73.66) (end 156.4025 73.66) (width 0.25) (layer "F.Cu") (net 23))
 (segment (start 156.4025 73.66) (end 155.5389 74.5236) (width 0.25) (layer "F.Cu") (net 23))
 (segment (start 141.5288 90.5256) (end 142.8708 89.1836) (width 0.25) (layer "F.Cu") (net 4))
 (segment (start 141.5288 91.8571) (end 141.5288 90.5256) (width 0.25) (layer "F.Cu") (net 4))
 (segment (start 142.8708 89.1836) (end 142.8708 87.4752) (width 0.25) (layer "F.Cu") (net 4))
 (segment (start 158.9998 82.3002) (end 144.1958 82.3002) (width 0.25) (layer "F.Cu") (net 6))
 (segment (start 144.1958 82.3002) (end 142.8708 80.9752) (width 0.25) (layer "F.Cu") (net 6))
 (segment (start 160.02 81.28) (end 158.9998 82.3002) (width 0.25) (layer "F.Cu") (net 6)))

